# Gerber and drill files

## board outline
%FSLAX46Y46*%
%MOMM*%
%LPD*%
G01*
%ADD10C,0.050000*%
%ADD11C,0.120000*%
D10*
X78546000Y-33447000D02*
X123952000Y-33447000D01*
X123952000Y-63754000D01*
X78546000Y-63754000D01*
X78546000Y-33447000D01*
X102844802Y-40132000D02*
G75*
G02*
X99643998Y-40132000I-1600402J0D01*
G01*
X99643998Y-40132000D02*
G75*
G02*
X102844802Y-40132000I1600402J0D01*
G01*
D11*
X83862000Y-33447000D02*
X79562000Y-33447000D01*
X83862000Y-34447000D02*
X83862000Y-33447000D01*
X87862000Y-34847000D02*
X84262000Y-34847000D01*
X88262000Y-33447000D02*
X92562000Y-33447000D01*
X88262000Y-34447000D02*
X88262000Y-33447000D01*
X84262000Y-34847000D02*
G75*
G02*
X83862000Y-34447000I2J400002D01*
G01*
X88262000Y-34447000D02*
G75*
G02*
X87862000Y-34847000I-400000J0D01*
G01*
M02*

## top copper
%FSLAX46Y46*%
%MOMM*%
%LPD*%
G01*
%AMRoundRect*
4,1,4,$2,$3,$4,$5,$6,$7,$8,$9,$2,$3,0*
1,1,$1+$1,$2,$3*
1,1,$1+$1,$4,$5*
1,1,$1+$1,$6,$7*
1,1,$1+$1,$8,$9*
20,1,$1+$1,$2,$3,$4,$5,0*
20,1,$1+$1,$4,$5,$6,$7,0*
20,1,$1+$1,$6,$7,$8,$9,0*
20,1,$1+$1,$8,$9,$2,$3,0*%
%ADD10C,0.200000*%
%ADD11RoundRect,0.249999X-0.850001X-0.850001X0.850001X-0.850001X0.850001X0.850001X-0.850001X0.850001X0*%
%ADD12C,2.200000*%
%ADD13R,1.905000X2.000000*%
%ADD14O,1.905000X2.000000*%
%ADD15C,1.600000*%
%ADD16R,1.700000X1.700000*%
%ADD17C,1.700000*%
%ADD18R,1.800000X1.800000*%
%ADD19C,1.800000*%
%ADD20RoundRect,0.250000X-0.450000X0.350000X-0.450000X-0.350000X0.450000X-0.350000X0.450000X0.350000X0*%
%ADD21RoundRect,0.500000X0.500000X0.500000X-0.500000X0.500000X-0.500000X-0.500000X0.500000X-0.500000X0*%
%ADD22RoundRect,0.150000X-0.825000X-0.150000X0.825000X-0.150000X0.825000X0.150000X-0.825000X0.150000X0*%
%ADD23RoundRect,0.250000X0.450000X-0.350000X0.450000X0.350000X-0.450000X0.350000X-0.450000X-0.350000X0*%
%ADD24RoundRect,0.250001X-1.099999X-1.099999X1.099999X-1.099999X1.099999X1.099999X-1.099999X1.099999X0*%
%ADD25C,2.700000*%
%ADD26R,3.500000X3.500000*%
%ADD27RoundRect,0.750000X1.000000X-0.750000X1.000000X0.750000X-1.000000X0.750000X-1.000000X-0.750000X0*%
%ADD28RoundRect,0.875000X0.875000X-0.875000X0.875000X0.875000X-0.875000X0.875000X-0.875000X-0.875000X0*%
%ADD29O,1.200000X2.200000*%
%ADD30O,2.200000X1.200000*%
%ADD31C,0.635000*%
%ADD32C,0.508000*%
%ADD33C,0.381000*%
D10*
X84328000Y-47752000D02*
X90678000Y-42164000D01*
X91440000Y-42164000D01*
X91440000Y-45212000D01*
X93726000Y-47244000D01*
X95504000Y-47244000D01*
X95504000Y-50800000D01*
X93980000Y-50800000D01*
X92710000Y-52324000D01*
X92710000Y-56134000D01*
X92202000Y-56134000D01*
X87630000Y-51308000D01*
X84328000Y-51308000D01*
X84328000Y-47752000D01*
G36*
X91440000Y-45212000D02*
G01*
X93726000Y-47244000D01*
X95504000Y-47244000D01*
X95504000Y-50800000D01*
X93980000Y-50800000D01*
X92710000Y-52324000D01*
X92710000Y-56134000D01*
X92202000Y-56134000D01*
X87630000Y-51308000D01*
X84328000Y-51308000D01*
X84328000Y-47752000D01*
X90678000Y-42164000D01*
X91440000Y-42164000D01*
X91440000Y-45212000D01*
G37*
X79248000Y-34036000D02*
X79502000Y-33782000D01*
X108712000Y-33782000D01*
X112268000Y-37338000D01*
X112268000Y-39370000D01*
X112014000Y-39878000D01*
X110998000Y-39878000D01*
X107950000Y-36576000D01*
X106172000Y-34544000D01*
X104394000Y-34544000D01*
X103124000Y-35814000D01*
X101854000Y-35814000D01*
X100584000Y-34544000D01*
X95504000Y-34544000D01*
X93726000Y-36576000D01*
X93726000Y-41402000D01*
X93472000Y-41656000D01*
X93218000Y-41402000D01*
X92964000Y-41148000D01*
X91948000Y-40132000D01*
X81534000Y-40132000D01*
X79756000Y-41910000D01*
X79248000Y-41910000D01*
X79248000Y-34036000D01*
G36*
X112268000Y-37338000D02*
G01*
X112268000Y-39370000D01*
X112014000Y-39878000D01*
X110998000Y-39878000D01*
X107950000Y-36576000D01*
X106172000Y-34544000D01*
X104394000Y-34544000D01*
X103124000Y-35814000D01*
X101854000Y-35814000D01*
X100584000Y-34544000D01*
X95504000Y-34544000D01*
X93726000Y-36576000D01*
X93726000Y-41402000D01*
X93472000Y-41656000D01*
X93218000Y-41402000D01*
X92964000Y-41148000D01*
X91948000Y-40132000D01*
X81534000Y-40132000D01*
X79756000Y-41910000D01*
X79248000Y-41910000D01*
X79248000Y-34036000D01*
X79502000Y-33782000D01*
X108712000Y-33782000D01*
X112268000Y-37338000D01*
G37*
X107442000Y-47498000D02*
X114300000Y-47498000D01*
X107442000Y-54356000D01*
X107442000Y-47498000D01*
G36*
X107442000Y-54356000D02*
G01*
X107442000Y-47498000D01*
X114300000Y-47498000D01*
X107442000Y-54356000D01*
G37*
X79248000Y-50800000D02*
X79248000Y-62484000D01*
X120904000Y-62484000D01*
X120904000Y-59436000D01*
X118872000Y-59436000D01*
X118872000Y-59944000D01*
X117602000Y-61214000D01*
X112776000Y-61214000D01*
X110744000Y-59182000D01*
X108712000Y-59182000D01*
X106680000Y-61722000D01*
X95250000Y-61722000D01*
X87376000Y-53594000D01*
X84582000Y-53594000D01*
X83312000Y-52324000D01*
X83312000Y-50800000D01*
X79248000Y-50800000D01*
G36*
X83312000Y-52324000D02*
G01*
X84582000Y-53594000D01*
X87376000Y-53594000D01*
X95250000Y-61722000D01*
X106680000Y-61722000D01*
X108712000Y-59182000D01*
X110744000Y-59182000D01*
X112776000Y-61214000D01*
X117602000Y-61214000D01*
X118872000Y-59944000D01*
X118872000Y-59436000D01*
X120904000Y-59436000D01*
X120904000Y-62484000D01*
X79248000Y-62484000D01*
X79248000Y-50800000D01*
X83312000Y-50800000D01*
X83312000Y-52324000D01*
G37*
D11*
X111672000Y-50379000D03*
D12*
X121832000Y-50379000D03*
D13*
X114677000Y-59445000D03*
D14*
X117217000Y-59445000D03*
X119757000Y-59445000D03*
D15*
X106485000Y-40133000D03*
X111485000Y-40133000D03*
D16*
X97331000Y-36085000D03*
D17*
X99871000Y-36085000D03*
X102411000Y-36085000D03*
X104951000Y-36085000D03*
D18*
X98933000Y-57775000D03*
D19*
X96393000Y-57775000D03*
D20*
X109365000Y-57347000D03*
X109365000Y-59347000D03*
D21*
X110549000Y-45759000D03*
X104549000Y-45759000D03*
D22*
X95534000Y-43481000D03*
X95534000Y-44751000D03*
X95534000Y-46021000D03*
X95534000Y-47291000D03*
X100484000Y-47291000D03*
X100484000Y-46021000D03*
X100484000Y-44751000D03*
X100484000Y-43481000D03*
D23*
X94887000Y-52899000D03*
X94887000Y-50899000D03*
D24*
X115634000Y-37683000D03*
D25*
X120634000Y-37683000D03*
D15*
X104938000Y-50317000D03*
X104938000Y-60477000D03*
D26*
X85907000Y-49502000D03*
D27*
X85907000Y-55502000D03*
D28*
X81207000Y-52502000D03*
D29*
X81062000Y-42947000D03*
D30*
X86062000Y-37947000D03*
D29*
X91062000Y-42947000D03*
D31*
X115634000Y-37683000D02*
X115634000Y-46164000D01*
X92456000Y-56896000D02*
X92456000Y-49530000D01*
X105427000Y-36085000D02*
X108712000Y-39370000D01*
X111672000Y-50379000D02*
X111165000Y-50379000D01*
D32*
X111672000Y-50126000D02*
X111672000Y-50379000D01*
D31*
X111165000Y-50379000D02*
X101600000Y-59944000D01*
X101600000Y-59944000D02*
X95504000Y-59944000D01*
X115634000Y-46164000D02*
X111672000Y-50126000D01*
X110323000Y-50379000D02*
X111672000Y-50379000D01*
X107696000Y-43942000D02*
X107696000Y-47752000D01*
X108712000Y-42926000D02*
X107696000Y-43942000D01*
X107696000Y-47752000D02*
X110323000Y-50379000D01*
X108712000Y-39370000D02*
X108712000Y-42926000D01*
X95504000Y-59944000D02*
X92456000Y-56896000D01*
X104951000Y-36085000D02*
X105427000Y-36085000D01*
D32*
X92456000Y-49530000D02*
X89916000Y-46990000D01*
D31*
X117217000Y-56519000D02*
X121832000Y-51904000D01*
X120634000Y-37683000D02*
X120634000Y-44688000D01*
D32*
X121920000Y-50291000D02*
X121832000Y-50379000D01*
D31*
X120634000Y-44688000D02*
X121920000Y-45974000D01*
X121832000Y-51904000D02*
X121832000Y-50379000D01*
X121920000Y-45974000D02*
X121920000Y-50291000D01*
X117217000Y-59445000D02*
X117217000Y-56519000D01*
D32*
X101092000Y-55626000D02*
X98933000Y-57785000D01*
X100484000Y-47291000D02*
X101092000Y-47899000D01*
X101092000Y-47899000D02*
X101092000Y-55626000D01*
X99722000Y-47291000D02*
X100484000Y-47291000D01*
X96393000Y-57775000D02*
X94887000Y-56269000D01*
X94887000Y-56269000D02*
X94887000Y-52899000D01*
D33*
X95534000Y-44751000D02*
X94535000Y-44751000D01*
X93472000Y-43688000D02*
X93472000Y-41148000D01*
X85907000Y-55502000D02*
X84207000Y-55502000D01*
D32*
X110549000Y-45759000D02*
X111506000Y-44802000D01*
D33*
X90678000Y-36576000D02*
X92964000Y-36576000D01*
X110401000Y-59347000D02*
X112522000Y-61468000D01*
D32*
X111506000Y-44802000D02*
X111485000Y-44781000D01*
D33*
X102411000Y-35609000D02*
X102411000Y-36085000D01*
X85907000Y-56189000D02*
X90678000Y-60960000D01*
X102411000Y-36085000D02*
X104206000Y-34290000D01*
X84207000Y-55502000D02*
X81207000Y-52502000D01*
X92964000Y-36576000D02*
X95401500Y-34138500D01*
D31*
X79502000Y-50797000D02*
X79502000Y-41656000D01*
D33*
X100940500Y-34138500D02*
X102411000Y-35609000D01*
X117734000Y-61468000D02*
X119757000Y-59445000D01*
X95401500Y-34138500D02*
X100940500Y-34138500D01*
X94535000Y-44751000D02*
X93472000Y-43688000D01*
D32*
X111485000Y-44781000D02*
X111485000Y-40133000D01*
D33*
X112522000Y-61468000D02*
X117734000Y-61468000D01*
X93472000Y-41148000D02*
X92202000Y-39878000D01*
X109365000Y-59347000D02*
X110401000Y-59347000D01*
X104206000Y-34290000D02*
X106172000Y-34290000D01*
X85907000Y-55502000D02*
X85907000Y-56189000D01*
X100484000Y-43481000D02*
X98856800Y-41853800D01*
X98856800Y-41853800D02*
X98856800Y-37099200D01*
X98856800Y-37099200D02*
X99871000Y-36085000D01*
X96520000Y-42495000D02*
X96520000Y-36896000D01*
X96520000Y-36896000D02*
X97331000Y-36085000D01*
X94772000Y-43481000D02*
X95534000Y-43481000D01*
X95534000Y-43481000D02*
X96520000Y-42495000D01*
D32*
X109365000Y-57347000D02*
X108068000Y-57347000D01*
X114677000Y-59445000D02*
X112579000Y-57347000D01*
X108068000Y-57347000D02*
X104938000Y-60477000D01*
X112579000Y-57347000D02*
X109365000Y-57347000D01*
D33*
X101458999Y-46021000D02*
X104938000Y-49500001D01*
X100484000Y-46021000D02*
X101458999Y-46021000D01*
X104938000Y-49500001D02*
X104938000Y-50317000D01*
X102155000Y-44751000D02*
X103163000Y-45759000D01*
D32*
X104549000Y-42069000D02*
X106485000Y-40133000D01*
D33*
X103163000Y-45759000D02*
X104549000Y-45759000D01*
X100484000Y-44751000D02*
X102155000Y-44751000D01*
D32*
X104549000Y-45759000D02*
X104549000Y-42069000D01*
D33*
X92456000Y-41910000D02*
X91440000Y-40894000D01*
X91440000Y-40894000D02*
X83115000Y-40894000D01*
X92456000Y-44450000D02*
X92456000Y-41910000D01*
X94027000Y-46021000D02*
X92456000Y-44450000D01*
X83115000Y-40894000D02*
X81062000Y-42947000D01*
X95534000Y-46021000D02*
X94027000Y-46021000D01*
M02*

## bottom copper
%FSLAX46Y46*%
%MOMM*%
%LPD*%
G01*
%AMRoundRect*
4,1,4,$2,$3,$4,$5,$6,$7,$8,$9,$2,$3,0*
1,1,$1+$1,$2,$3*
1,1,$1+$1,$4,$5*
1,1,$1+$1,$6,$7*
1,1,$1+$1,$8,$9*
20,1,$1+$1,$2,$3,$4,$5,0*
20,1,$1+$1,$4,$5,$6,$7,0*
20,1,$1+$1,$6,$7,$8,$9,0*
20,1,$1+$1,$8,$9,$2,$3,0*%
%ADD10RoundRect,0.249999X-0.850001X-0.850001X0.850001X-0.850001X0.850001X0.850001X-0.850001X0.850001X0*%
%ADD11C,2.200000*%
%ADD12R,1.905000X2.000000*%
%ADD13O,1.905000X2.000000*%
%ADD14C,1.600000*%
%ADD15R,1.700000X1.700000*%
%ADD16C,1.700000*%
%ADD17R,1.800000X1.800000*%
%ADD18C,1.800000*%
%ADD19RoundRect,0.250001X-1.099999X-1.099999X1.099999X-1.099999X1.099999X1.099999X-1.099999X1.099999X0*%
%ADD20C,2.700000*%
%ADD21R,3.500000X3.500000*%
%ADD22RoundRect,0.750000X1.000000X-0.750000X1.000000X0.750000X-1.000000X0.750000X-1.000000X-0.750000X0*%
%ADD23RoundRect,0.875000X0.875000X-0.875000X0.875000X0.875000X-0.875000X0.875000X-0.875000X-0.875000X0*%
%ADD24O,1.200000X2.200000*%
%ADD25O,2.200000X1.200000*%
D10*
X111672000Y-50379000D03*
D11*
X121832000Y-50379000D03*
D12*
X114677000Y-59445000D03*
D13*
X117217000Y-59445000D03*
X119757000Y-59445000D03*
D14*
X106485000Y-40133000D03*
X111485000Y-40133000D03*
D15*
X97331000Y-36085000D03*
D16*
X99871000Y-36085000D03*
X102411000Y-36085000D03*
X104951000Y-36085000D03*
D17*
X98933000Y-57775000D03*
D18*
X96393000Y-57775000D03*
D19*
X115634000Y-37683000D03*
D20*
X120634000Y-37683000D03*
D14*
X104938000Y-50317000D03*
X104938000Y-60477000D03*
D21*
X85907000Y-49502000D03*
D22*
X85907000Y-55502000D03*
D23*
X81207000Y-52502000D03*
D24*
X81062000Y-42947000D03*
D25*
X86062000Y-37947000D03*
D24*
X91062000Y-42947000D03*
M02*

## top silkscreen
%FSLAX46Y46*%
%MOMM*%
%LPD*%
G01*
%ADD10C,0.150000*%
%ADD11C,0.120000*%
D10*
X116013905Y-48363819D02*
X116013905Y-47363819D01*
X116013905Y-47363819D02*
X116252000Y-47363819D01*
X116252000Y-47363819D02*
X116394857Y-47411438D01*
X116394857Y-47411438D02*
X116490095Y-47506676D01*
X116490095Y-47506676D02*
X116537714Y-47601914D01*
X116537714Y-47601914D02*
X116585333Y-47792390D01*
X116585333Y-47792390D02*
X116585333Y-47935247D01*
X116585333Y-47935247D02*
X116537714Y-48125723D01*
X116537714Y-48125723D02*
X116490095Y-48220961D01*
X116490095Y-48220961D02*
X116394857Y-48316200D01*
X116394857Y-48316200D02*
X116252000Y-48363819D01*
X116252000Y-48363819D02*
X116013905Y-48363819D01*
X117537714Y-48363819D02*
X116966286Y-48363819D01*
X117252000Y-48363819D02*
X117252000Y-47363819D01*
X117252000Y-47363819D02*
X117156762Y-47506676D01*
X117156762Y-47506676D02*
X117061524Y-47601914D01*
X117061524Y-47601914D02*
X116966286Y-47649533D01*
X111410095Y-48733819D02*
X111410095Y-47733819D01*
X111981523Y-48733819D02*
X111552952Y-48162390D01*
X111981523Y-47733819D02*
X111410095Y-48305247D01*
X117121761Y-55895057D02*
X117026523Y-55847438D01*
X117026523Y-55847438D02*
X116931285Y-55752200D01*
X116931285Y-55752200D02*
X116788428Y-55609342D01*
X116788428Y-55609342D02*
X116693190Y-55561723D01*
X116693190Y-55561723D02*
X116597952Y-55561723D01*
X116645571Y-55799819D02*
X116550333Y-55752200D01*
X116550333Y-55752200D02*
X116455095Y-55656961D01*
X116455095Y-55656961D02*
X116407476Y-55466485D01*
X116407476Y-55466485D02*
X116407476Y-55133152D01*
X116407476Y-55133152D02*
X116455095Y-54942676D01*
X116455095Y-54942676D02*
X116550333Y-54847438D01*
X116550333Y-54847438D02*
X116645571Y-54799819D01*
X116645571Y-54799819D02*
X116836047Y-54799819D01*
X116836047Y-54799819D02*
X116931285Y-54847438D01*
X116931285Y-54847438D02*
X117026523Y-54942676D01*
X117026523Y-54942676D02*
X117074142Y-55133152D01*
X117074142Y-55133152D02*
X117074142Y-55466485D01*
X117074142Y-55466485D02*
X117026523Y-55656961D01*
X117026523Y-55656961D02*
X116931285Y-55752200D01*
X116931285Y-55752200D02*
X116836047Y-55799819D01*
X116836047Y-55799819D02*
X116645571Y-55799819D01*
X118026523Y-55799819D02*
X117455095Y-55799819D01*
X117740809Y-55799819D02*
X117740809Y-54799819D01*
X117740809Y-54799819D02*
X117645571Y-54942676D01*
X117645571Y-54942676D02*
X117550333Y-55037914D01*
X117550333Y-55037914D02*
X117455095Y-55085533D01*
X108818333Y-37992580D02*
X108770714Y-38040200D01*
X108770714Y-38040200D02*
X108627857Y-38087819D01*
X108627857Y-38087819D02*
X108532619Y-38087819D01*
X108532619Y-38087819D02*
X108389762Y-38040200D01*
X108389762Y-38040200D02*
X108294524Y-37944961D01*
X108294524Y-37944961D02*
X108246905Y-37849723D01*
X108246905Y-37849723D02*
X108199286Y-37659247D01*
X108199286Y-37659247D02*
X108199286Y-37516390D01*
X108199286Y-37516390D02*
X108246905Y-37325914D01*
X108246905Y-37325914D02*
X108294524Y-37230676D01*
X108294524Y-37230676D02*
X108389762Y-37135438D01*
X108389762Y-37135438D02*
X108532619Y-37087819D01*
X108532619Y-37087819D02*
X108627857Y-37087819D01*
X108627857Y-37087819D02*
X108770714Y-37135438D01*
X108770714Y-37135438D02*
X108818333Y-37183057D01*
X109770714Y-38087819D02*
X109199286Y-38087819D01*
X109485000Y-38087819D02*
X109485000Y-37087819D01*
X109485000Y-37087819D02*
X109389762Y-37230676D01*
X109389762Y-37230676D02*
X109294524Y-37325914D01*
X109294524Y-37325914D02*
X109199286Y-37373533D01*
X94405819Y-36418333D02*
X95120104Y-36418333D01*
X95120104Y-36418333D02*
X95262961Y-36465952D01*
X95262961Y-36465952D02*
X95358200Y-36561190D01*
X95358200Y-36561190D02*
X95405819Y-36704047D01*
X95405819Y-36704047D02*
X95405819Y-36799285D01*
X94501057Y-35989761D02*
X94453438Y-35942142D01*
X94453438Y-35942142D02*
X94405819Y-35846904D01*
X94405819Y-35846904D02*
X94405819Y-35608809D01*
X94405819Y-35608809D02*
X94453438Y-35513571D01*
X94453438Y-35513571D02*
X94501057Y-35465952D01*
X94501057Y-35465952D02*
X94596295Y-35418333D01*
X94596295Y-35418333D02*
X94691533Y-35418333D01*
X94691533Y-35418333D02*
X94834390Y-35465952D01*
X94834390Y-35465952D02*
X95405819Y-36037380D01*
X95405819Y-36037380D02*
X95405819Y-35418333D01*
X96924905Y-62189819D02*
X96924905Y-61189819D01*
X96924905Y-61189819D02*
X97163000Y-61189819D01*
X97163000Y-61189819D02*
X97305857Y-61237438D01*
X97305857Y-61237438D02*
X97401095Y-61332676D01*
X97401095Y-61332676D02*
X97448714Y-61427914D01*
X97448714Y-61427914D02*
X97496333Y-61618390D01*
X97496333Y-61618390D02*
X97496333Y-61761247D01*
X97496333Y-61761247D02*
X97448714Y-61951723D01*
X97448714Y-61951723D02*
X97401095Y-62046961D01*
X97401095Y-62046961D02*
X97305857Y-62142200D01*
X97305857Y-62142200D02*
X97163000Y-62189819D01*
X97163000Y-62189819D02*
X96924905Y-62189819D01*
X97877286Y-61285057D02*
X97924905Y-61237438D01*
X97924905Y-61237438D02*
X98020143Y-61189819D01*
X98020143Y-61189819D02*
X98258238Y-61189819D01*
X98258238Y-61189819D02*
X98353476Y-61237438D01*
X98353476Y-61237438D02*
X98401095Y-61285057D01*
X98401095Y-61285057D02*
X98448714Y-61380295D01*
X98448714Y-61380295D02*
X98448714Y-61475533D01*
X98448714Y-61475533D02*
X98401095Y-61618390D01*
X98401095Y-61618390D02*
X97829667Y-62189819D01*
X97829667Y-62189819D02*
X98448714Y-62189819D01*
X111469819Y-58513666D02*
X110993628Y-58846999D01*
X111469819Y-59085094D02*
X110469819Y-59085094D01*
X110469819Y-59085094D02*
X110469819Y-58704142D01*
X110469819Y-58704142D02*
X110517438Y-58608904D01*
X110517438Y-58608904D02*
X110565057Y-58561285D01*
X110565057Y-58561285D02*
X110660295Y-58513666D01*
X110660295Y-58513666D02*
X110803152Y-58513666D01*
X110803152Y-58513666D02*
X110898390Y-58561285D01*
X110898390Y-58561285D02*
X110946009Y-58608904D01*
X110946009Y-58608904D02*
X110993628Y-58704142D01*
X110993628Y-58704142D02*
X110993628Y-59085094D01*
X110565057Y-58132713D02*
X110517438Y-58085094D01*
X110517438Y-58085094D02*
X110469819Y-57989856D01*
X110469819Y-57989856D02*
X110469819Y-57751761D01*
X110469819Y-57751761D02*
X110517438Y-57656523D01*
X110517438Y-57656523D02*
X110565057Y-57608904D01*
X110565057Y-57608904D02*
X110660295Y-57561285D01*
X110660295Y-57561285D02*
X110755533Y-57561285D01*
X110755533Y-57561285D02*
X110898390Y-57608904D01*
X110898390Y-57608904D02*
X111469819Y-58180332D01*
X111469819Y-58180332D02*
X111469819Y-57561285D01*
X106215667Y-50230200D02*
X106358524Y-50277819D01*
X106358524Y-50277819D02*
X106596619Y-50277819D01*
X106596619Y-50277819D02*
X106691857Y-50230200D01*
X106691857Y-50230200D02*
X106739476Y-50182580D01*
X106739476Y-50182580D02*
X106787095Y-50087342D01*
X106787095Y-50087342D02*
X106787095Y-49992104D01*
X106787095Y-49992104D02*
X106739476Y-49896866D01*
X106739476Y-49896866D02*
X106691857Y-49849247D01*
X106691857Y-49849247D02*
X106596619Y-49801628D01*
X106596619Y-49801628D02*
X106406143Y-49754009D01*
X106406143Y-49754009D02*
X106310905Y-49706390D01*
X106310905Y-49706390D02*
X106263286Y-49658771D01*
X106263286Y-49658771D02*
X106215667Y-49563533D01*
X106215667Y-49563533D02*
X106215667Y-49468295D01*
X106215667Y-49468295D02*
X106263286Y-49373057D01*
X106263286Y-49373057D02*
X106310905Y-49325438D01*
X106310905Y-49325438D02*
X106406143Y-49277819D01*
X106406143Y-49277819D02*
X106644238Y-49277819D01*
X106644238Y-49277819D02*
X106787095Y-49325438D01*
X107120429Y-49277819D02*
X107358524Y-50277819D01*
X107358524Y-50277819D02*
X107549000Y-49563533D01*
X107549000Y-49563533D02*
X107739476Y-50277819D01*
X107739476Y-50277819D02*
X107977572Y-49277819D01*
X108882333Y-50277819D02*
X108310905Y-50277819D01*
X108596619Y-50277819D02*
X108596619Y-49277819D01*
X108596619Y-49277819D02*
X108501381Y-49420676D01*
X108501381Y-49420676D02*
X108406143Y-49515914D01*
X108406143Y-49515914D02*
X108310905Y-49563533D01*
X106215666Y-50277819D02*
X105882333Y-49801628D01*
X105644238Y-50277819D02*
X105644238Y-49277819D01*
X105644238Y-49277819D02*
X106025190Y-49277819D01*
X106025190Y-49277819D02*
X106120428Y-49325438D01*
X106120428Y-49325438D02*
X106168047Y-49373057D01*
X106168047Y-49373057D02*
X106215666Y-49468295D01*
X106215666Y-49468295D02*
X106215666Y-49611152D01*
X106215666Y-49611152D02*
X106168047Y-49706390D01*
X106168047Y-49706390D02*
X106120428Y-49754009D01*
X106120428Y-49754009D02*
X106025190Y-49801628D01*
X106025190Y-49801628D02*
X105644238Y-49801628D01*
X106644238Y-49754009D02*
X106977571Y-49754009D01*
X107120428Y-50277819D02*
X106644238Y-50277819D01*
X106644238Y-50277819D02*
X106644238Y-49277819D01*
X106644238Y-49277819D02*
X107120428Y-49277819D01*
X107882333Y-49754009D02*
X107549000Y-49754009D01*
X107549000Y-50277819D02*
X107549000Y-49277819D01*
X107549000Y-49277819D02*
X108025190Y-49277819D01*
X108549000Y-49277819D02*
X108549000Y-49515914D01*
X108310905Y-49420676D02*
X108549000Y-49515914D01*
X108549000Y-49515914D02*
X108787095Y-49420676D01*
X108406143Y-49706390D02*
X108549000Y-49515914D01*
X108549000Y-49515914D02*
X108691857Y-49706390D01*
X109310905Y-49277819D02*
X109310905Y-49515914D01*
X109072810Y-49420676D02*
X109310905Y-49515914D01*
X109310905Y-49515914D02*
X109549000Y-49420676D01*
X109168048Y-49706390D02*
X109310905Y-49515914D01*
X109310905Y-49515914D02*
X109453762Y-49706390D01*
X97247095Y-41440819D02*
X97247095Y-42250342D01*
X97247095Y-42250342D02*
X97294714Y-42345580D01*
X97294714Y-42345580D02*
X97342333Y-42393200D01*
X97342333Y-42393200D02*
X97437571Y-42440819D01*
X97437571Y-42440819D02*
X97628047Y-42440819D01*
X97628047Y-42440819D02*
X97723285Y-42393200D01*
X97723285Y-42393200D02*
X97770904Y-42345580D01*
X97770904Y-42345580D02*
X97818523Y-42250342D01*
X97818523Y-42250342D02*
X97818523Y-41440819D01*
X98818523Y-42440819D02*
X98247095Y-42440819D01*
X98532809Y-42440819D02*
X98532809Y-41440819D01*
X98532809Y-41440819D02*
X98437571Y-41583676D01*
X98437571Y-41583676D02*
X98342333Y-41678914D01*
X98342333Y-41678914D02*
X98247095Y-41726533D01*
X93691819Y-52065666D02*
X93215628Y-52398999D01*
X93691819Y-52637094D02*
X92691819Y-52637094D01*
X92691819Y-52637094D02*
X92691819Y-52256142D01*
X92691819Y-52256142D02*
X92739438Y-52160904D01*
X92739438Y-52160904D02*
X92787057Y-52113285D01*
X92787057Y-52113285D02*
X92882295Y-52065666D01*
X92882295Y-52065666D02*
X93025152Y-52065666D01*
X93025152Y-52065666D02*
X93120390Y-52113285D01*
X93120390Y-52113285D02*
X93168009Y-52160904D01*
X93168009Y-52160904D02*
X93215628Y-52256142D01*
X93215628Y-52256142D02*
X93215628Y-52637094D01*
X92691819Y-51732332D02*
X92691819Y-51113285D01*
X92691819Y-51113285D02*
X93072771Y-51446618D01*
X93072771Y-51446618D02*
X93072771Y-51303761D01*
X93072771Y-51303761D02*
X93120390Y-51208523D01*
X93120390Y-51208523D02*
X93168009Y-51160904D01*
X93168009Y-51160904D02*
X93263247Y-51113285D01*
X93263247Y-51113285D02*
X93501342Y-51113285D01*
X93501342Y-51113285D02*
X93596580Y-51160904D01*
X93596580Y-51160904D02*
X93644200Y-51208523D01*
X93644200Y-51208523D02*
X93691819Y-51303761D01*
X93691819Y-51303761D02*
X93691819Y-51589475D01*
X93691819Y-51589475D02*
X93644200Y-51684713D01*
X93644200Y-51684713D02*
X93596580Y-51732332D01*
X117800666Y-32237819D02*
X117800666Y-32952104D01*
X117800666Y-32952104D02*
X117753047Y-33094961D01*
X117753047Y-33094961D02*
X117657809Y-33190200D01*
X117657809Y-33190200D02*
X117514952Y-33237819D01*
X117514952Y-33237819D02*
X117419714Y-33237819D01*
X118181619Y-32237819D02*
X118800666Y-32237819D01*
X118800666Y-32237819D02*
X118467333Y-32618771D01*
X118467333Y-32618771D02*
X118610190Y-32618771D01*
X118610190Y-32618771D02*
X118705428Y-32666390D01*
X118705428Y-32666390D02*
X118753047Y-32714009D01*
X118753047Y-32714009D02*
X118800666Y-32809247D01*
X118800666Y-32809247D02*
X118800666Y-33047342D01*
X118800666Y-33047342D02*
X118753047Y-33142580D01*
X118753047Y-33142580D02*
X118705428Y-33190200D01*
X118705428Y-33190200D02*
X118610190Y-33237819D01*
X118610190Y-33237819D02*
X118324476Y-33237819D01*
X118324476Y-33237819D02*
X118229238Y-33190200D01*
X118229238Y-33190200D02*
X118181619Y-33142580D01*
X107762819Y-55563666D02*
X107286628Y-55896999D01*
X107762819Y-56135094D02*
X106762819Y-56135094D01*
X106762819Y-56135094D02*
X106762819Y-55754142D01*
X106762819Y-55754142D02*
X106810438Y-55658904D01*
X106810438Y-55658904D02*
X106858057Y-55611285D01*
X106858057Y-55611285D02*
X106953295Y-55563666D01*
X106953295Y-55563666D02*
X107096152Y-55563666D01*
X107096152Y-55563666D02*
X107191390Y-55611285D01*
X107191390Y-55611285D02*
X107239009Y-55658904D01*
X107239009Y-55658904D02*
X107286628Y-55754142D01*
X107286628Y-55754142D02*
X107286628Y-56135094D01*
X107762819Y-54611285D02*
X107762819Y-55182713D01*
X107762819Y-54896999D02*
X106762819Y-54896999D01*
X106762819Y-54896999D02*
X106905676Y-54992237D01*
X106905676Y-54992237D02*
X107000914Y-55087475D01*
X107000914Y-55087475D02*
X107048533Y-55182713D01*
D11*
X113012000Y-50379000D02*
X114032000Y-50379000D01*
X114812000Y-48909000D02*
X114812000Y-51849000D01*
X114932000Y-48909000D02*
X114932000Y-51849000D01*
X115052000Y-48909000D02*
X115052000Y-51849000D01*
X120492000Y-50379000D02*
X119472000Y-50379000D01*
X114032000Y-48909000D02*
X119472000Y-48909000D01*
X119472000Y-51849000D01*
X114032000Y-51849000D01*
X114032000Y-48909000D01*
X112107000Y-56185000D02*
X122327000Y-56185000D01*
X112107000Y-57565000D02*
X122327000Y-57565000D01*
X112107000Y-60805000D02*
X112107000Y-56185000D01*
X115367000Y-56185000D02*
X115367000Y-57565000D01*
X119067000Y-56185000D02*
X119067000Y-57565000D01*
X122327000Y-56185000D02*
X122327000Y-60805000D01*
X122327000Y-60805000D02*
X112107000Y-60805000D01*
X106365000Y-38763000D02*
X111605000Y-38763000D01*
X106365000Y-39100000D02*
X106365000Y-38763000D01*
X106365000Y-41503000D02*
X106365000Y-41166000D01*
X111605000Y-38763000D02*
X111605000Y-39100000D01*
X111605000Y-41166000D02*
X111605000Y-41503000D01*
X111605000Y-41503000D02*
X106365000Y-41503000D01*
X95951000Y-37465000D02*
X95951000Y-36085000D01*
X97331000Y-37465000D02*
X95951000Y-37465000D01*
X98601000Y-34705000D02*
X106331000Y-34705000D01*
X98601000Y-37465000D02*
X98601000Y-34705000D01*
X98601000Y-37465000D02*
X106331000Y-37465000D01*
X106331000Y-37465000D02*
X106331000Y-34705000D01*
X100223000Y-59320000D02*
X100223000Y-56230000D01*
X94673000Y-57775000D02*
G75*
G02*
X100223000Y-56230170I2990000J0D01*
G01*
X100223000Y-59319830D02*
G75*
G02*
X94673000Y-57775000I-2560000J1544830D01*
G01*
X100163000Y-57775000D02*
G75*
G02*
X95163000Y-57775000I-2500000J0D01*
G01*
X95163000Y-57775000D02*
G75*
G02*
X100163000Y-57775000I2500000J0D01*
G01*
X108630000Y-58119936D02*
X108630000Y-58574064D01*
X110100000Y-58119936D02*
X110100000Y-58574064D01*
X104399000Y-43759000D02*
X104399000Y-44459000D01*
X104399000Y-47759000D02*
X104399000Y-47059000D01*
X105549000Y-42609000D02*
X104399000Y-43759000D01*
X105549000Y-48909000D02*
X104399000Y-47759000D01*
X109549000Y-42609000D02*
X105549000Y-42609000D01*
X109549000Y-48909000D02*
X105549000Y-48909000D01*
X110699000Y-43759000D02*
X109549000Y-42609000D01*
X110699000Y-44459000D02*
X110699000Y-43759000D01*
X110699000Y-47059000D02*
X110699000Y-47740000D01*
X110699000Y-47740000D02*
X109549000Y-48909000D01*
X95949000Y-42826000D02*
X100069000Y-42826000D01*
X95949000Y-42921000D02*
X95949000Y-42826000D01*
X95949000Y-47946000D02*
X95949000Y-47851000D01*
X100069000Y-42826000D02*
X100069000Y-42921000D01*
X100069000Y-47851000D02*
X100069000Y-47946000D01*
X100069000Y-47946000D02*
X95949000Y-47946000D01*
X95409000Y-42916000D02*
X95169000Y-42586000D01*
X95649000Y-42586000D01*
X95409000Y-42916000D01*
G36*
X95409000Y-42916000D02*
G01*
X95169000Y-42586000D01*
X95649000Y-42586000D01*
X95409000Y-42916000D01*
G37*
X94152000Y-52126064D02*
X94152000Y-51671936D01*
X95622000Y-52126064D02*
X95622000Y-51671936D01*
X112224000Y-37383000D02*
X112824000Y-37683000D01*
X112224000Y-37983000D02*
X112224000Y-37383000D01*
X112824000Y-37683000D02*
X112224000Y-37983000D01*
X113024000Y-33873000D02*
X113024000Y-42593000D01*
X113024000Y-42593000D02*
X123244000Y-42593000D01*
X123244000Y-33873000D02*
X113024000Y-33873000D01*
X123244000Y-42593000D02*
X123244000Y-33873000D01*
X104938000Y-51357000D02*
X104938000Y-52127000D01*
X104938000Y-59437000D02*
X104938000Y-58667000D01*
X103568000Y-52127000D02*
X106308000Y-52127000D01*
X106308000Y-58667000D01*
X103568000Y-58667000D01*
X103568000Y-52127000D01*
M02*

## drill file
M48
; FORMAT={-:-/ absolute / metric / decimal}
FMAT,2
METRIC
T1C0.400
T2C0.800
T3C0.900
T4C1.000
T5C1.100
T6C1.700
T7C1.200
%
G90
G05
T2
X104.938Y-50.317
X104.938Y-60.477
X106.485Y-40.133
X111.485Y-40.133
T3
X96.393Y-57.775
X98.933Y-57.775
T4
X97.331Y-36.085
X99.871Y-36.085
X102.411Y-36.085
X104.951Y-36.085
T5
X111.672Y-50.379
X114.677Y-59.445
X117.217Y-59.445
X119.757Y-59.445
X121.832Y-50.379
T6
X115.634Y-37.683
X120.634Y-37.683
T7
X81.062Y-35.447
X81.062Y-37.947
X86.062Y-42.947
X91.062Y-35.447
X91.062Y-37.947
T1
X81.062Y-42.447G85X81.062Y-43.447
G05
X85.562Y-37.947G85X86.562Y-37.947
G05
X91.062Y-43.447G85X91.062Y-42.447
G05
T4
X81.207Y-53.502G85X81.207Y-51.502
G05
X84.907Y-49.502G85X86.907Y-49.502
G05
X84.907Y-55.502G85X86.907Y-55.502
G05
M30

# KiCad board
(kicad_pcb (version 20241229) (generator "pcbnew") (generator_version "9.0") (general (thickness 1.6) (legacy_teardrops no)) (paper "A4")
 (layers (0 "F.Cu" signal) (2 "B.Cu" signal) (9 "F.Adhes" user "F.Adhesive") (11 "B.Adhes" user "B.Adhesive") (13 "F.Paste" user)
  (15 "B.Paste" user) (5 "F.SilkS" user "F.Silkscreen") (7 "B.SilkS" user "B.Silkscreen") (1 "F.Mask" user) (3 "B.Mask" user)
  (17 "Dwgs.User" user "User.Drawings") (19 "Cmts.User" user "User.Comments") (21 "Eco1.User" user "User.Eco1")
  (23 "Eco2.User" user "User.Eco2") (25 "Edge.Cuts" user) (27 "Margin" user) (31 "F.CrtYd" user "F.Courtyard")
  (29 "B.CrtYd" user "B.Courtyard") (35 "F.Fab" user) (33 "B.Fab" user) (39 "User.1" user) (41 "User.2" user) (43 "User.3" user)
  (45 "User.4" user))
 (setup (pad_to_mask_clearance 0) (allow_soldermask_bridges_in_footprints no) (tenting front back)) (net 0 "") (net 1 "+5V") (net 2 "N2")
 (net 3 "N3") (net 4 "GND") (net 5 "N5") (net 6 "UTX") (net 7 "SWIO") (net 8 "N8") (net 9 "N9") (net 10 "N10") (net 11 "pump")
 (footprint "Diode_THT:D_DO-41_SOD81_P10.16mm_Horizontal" (layer "F.Cu") (at 111.672 50.379)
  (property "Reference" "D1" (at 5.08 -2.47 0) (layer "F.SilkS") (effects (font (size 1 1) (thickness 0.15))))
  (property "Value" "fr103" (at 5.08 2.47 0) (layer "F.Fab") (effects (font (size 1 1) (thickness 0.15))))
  (fp_line (start 1.34 0) (end 2.36 0) (stroke (width 0.12) (type solid)) (layer "F.SilkS"))
  (fp_line (start 3.14 -1.47) (end 3.14 1.47) (stroke (width 0.12) (type solid)) (layer "F.SilkS"))
  (fp_line (start 3.26 -1.47) (end 3.26 1.47) (stroke (width 0.12) (type solid)) (layer "F.SilkS"))
  (fp_line (start 3.38 -1.47) (end 3.38 1.47) (stroke (width 0.12) (type solid)) (layer "F.SilkS"))
  (fp_line (start 8.82 0) (end 7.8 0) (stroke (width 0.12) (type solid)) (layer "F.SilkS"))
  (fp_rect (start 2.36 -1.47) (end 7.8 1.47) (stroke (width 0.12) (type solid)) (fill no) (layer "F.SilkS"))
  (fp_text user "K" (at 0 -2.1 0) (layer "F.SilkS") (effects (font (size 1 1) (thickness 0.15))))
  (pad "1" thru_hole roundrect (at 0 0) (size 2.2 2.2) (drill 1.1) (layers "*.Cu" "*.Mask") (remove_unused_layers no)
   (roundrect_rratio 0.113636) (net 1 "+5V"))
  (pad "2" thru_hole circle (at 10.16 0) (size 2.2 2.2) (drill 1.1) (layers "*.Cu" "*.Mask") (remove_unused_layers no) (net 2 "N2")))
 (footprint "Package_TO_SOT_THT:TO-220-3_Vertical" (layer "F.Cu") (at 114.677 59.445)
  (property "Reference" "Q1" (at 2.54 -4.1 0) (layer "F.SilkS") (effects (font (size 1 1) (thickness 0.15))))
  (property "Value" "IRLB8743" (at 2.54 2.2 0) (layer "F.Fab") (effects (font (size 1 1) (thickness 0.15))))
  (fp_line (start -2.57 -3.26) (end 7.65 -3.26) (stroke (width 0.12) (type solid)) (layer "F.SilkS"))
  (fp_line (start -2.57 -1.88) (end 7.65 -1.88) (stroke (width 0.12) (type solid)) (layer "F.SilkS"))
  (fp_line (start -2.57 1.36) (end -2.57 -3.26) (stroke (width 0.12) (type solid)) (layer "F.SilkS"))
  (fp_line (start 0.69 -3.26) (end 0.69 -1.88) (stroke (width 0.12) (type solid)) (layer "F.SilkS"))
  (fp_line (start 4.39 -3.26) (end 4.39 -1.88) (stroke (width 0.12) (type solid)) (layer "F.SilkS"))
  (fp_line (start 7.65 -3.26) (end 7.65 1.36) (stroke (width 0.12) (type solid)) (layer "F.SilkS"))
  (fp_line (start 7.65 1.36) (end -2.57 1.36) (stroke (width 0.12) (type solid)) (layer "F.SilkS"))
  (pad "1" thru_hole rect (at 0 0) (size 1.905 2) (drill 1.1) (layers "*.Cu" "*.Mask") (remove_unused_layers no) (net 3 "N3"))
  (pad "2" thru_hole oval (at 2.54 0) (size 1.905 2) (drill 1.1) (layers "*.Cu" "*.Mask") (remove_unused_layers no) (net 2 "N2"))
  (pad "3" thru_hole oval (at 5.08 0) (size 1.905 2) (drill 1.1) (layers "*.Cu" "*.Mask") (remove_unused_layers no) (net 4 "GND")))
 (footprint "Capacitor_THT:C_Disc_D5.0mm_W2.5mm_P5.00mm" (layer "F.Cu") (at 106.485 40.133)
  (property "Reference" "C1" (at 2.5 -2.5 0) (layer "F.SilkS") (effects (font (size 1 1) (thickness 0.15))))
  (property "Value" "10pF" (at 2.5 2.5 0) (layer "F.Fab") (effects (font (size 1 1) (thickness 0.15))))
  (fp_line (start -0.12 -1.37) (end 5.12 -1.37) (stroke (width 0.12) (type solid)) (layer "F.SilkS"))
  (fp_line (start -0.12 -1.033) (end -0.12 -1.37) (stroke (width 0.12) (type solid)) (layer "F.SilkS"))
  (fp_line (start -0.12 1.37) (end -0.12 1.033) (stroke (width 0.12) (type solid)) (layer "F.SilkS"))
  (fp_line (start 5.12 -1.37) (end 5.12 -1.033) (stroke (width 0.12) (type solid)) (layer "F.SilkS"))
  (fp_line (start 5.12 1.033) (end 5.12 1.37) (stroke (width 0.12) (type solid)) (layer "F.SilkS"))
  (fp_line (start 5.12 1.37) (end -0.12 1.37) (stroke (width 0.12) (type solid)) (layer "F.SilkS"))
  (pad "1" thru_hole circle (at 0 0) (size 1.6 1.6) (drill 0.8) (layers "*.Cu" "*.Mask") (remove_unused_layers no) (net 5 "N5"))
  (pad "2" thru_hole circle (at 5 0) (size 1.6 1.6) (drill 0.8) (layers "*.Cu" "*.Mask") (remove_unused_layers no) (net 4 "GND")))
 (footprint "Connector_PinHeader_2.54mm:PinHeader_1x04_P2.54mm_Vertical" (layer "F.Cu") (at 97.331 36.085 90)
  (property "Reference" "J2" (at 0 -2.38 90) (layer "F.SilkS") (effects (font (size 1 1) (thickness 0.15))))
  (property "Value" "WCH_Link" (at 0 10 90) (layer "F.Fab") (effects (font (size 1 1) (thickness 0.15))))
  (fp_line (start -1.38 -1.38) (end 0 -1.38) (stroke (width 0.12) (type solid)) (layer "F.SilkS"))
  (fp_line (start -1.38 0) (end -1.38 -1.38) (stroke (width 0.12) (type solid)) (layer "F.SilkS"))
  (fp_line (start 1.38 1.27) (end 1.38 9) (stroke (width 0.12) (type solid)) (layer "F.SilkS"))
  (fp_line (start -1.38 1.27) (end 1.38 1.27) (stroke (width 0.12) (type solid)) (layer "F.SilkS"))
  (fp_line (start -1.38 1.27) (end -1.38 9) (stroke (width 0.12) (type solid)) (layer "F.SilkS"))
  (fp_line (start -1.38 9) (end 1.38 9) (stroke (width 0.12) (type solid)) (layer "F.SilkS"))
  (pad "1" thru_hole rect (at 0 0 90) (size 1.7 1.7) (drill 1) (layers "*.Cu" "*.Mask") (remove_unused_layers no) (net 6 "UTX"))
  (pad "2" thru_hole circle (at 0 2.54 90) (size 1.7 1.7) (drill 1) (layers "*.Cu" "*.Mask") (remove_unused_layers no) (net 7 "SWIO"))
  (pad "3" thru_hole circle (at 0 5.08 90) (size 1.7 1.7) (drill 1) (layers "*.Cu" "*.Mask") (remove_unused_layers no) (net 4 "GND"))
  (pad "4" thru_hole circle (at 0 7.62 90) (size 1.7 1.7) (drill 1) (layers "*.Cu" "*.Mask") (remove_unused_layers no) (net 1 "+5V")))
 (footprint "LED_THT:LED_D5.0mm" (layer "F.Cu") (at 98.933 57.775 180)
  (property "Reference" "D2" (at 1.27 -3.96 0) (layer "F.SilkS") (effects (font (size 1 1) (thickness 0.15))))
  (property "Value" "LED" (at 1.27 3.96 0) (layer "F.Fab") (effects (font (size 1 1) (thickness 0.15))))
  (fp_line (start -1.29 -1.545) (end -1.29 1.545) (stroke (width 0.12) (type solid)) (layer "F.SilkS"))
  (fp_arc (start 4.26 0) (mid 2.071779 2.880495) (end -1.29 1.54483) (stroke (width 0.12) (type solid)) (layer "F.SilkS"))
  (fp_arc (start -1.29 -1.54483) (mid 2.071779 -2.880495) (end 4.26 0) (stroke (width 0.12) (type solid)) (layer "F.SilkS"))
  (fp_circle (center 1.27 0) (end 3.77 0) (stroke (width 0.12) (type solid)) (fill no) (layer "F.SilkS"))
  (pad "1" thru_hole rect (at 0 0 180) (size 1.8 1.8) (drill 0.9) (layers "*.Cu" "*.Mask") (remove_unused_layers no) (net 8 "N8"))
  (pad "2" thru_hole circle (at 2.54 0 180) (size 1.8 1.8) (drill 0.9) (layers "*.Cu" "*.Mask") (remove_unused_layers no) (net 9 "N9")))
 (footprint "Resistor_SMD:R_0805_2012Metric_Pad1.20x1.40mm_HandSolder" (layer "F.Cu") (at 109.365 58.347 -90)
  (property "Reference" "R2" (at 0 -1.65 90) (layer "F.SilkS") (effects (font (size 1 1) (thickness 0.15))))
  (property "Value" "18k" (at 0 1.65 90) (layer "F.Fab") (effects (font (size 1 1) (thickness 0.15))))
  (fp_line (start -0.227064 0.735) (end 0.227064 0.735) (stroke (width 0.12) (type solid)) (layer "F.SilkS"))
  (fp_line (start -0.227064 -0.735) (end 0.227064 -0.735) (stroke (width 0.12) (type solid)) (layer "F.SilkS"))
  (pad "1" smd roundrect (at -1 0 270) (size 1.2 1.4) (layers "F.Cu" "F.Mask" "F.Paste") (roundrect_rratio 0.208333) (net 3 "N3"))
  (pad "2" smd roundrect (at 1 0 270) (size 1.2 1.4) (layers "F.Cu" "F.Mask" "F.Paste") (roundrect_rratio 0.208333) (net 4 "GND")))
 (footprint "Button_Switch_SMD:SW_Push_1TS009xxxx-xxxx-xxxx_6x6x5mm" (layer "F.Cu") (at 107.549 45.759 180)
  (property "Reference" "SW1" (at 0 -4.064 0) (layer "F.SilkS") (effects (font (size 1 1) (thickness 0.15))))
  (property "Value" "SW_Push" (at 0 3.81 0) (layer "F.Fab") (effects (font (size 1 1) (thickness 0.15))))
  (fp_line (start 3.15 2) (end 3.15 1.3) (stroke (width 0.12) (type default)) (layer "F.SilkS"))
  (fp_line (start 3.15 -2) (end 3.15 -1.3) (stroke (width 0.12) (type default)) (layer "F.SilkS"))
  (fp_line (start 2 3.15) (end 3.15 2) (stroke (width 0.12) (type default)) (layer "F.SilkS"))
  (fp_line (start 2 -3.15) (end 3.15 -2) (stroke (width 0.12) (type default)) (layer "F.SilkS"))
  (fp_line (start -2 3.15) (end 2 3.15) (stroke (width 0.12) (type default)) (layer "F.SilkS"))
  (fp_line (start -2 -3.15) (end 2 -3.15) (stroke (width 0.12) (type default)) (layer "F.SilkS"))
  (fp_line (start -3.15 2) (end -2 3.15) (stroke (width 0.12) (type default)) (layer "F.SilkS"))
  (fp_line (start -3.15 1.3) (end -3.15 2) (stroke (width 0.12) (type default)) (layer "F.SilkS"))
  (fp_line (start -3.15 -1.3) (end -3.15 -1.981) (stroke (width 0.12) (type default)) (layer "F.SilkS"))
  (fp_line (start -3.15 -1.981) (end -2 -3.15) (stroke (width 0.12) (type default)) (layer "F.SilkS"))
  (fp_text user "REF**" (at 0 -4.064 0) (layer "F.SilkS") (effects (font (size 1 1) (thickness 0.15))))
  (pad "1" smd roundrect (at -3 0 180) (size 2 2) (layers "F.Cu" "F.Mask" "F.Paste") (roundrect_rratio 0.25) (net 4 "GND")
   (thermal_bridge_angle 45))
  (pad "2" smd roundrect (at 3 0 180) (size 2 2) (layers "F.Cu" "F.Mask" "F.Paste") (roundrect_rratio 0.25) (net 5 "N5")
   (thermal_bridge_angle 45)))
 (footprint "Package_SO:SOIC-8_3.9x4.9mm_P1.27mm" (layer "F.Cu") (at 98.009 45.386)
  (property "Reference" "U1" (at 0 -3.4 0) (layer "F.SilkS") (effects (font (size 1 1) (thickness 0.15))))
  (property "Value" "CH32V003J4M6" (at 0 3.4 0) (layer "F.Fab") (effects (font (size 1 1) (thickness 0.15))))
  (fp_line (start -2.06 -2.56) (end 2.06 -2.56) (stroke (width 0.12) (type solid)) (layer "F.SilkS"))
  (fp_line (start -2.06 -2.465) (end -2.06 -2.56) (stroke (width 0.12) (type solid)) (layer "F.SilkS"))
  (fp_line (start -2.06 2.56) (end -2.06 2.465) (stroke (width 0.12) (type solid)) (layer "F.SilkS"))
  (fp_line (start 2.06 -2.56) (end 2.06 -2.465) (stroke (width 0.12) (type solid)) (layer "F.SilkS"))
  (fp_line (start 2.06 2.465) (end 2.06 2.56) (stroke (width 0.12) (type solid)) (layer "F.SilkS"))
  (fp_line (start 2.06 2.56) (end -2.06 2.56) (stroke (width 0.12) (type solid)) (layer "F.SilkS"))
  (fp_poly (pts (xy -2.6 -2.47) (xy -2.84 -2.8) (xy -2.36 -2.8)) (stroke (width 0.12) (type solid)) (fill yes) (layer "F.SilkS"))
  (pad "1" smd roundrect (at -2.475 -1.905) (size 1.95 0.6) (layers "F.Cu" "F.Mask" "F.Paste") (roundrect_rratio 0.25) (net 6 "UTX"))
  (pad "2" smd roundrect (at -2.475 -0.635) (size 1.95 0.6) (layers "F.Cu" "F.Mask" "F.Paste") (roundrect_rratio 0.25) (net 4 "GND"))
  (pad "3" smd roundrect (at -2.475 0.635) (size 1.95 0.6) (layers "F.Cu" "F.Mask" "F.Paste") (roundrect_rratio 0.25) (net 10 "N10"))
  (pad "4" smd roundrect (at -2.475 1.905) (size 1.95 0.6) (layers "F.Cu" "F.Mask" "F.Paste") (roundrect_rratio 0.25) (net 1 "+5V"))
  (pad "5" smd roundrect (at 2.475 1.905) (size 1.95 0.6) (layers "F.Cu" "F.Mask" "F.Paste") (roundrect_rratio 0.25) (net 8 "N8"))
  (pad "6" smd roundrect (at 2.475 0.635) (size 1.95 0.6) (layers "F.Cu" "F.Mask" "F.Paste") (roundrect_rratio 0.25) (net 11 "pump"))
  (pad "7" smd roundrect (at 2.475 -0.635) (size 1.95 0.6) (layers "F.Cu" "F.Mask" "F.Paste") (roundrect_rratio 0.25) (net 5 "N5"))
  (pad "8" smd roundrect (at 2.475 -1.905) (size 1.95 0.6) (layers "F.Cu" "F.Mask" "F.Paste") (roundrect_rratio 0.25) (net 7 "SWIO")))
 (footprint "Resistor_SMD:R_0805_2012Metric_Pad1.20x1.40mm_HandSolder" (layer "F.Cu") (at 94.887 51.899 90)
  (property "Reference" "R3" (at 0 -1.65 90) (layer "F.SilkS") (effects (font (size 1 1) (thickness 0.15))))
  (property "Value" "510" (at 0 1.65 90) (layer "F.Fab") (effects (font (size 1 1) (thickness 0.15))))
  (fp_line (start -0.227064 -0.735) (end 0.227064 -0.735) (stroke (width 0.12) (type solid)) (layer "F.SilkS"))
  (fp_line (start -0.227064 0.735) (end 0.227064 0.735) (stroke (width 0.12) (type solid)) (layer "F.SilkS"))
  (pad "1" smd roundrect (at -1 0 90) (size 1.2 1.4) (layers "F.Cu" "F.Mask" "F.Paste") (roundrect_rratio 0.208333) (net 9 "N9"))
  (pad "2" smd roundrect (at 1 0 90) (size 1.2 1.4) (layers "F.Cu" "F.Mask" "F.Paste") (roundrect_rratio 0.208333) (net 1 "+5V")))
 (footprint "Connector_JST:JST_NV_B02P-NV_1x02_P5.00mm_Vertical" (layer "F.Cu") (at 115.634 37.683)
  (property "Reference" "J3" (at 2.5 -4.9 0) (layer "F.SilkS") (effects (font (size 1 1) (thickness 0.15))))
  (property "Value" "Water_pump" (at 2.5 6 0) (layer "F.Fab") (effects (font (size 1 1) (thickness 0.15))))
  (fp_line (start -3.41 -0.3) (end -2.81 0) (stroke (width 0.12) (type solid)) (layer "F.SilkS"))
  (fp_line (start -3.41 0.3) (end -3.41 -0.3) (stroke (width 0.12) (type solid)) (layer "F.SilkS"))
  (fp_line (start -2.81 0) (end -3.41 0.3) (stroke (width 0.12) (type solid)) (layer "F.SilkS"))
  (fp_line (start -2.61 -3.81) (end -2.61 4.91) (stroke (width 0.12) (type solid)) (layer "F.SilkS"))
  (fp_line (start -2.61 4.91) (end 7.61 4.91) (stroke (width 0.12) (type solid)) (layer "F.SilkS"))
  (fp_line (start 7.61 -3.81) (end -2.61 -3.81) (stroke (width 0.12) (type solid)) (layer "F.SilkS"))
  (fp_line (start 7.61 4.91) (end 7.61 -3.81) (stroke (width 0.12) (type solid)) (layer "F.SilkS"))
  (pad "1" thru_hole roundrect (at 0 0) (size 2.7 2.7) (drill 1.7) (layers "*.Cu" "*.Mask") (remove_unused_layers no)
   (roundrect_rratio 0.092593) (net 1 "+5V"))
  (pad "2" thru_hole circle (at 5 0) (size 2.7 2.7) (drill 1.7) (layers "*.Cu" "*.Mask") (remove_unused_layers no) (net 2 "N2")))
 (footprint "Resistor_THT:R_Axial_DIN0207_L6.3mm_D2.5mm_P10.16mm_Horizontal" (layer "F.Cu") (at 104.938 50.317 -90)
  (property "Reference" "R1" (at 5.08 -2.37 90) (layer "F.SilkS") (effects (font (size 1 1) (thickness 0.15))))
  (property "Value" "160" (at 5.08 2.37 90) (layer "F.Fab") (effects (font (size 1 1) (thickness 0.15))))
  (fp_line (start 1.04 0) (end 1.81 0) (stroke (width 0.12) (type solid)) (layer "F.SilkS"))
  (fp_line (start 9.12 0) (end 8.35 0) (stroke (width 0.12) (type solid)) (layer "F.SilkS"))
  (fp_rect (start 1.81 -1.37) (end 8.35 1.37) (stroke (width 0.12) (type solid)) (fill no) (layer "F.SilkS"))
  (pad "1" thru_hole circle (at 0 0 270) (size 1.6 1.6) (drill 0.8) (layers "*.Cu" "*.Mask") (remove_unused_layers no) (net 11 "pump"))
  (pad "2" thru_hole circle (at 10.16 0 270) (size 1.6 1.6) (drill 0.8) (layers "*.Cu" "*.Mask") (remove_unused_layers no) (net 3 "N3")))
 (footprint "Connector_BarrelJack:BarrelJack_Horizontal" (layer "B.Cu") (at 85.907 49.502 90)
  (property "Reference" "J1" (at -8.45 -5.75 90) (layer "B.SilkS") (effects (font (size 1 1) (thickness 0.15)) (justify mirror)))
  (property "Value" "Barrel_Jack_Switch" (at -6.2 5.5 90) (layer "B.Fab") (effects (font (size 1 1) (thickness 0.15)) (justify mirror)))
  (pad "1" thru_hole rect (at 0 0 90) (size 3.5 3.5) (drill oval 1 3) (layers "*.Cu" "*.Mask") (remove_unused_layers no) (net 1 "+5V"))
  (pad "2" thru_hole roundrect (at -6 0 90) (size 3 3.5) (drill oval 1 3) (layers "*.Cu" "*.Mask") (remove_unused_layers no)
   (roundrect_rratio 0.25) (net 4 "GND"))
  (pad "3" thru_hole roundrect (at -3 -4.7 90) (size 3.5 3.5) (drill oval 3 1) (layers "*.Cu" "*.Mask") (remove_unused_layers no)
   (roundrect_rratio 0.25) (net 4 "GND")))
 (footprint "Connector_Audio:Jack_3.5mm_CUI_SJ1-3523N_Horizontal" (layer "B.Cu") (at 86.062 37.947)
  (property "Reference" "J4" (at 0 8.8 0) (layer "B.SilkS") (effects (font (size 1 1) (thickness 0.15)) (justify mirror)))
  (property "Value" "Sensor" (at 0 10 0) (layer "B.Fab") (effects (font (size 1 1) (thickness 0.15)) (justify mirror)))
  (fp_line (start -2.2 -4.5) (end -6.5 -4.5) (stroke (width 0.12) (type solid)) (layer "Edge.Cuts"))
  (fp_line (start -2.2 -3.5) (end -2.2 -4.5) (stroke (width 0.12) (type solid)) (layer "Edge.Cuts"))
  (fp_line (start 1.8 -3.1) (end -1.8 -3.1) (stroke (width 0.12) (type solid)) (layer "Edge.Cuts"))
  (fp_line (start 2.2 -4.5) (end 6.5 -4.5) (stroke (width 0.12) (type solid)) (layer "Edge.Cuts"))
  (fp_line (start 2.2 -3.5) (end 2.2 -4.5) (stroke (width 0.12) (type solid)) (layer "Edge.Cuts"))
  (fp_arc (start -1.8 -3.1) (mid -2.082842 -3.217158) (end -2.2 -3.5) (stroke (width 0.12) (type solid)) (layer "Edge.Cuts"))
  (fp_arc (start 2.2 -3.5) (mid 2.082843 -3.217157) (end 1.8 -3.1) (stroke (width 0.12) (type solid)) (layer "Edge.Cuts"))
  (pad "" np_thru_hole circle (at -5 -2.5) (size 1.2 1.2) (drill 1.2) (layers "*.Cu" "*.Mask"))
  (pad "" np_thru_hole circle (at -5 0) (size 1.2 1.2) (drill 1.2) (layers "*.Cu" "*.Mask"))
  (pad "" np_thru_hole circle (at 0 5) (size 1.2 1.2) (drill 1.2) (layers "*.Cu" "*.Mask"))
  (pad "" np_thru_hole circle (at 5 -2.5) (size 1.2 1.2) (drill 1.2) (layers "*.Cu" "*.Mask"))
  (pad "" np_thru_hole circle (at 5 0) (size 1.2 1.2) (drill 1.2) (layers "*.Cu" "*.Mask"))
  (pad "R" thru_hole oval (at -5 5) (size 1.2 2.2) (drill oval 0.4 1.4) (layers "*.Cu" "*.Mask") (remove_unused_layers no) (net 10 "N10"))
  (pad "S" thru_hole oval (at 0 0) (size 2.2 1.2) (drill oval 1.4 0.4) (layers "*.Cu" "*.Mask") (remove_unused_layers no) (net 4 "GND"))
  (pad "T" thru_hole oval (at 5 5 180) (size 1.2 2.2) (drill oval 0.4 1.4) (layers "*.Cu" "*.Mask") (remove_unused_layers no) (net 1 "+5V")))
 (gr_poly
  (pts (xy 84.328 47.752) (xy 90.678 42.164) (xy 91.44 42.164) (xy 91.44 45.212) (xy 93.726 47.244) (xy 95.504 47.244) (xy 95.504 50.8)
   (xy 93.98 50.8) (xy 92.71 52.324) (xy 92.71 56.134) (xy 92.202 56.134) (xy 87.63 51.308) (xy 84.328 51.308))
  (stroke (width 0.2) (type solid)) (fill yes) (layer "F.Cu") (net 1))
 (gr_poly
  (pts (xy 79.248 34.036) (xy 79.502 33.782) (xy 108.712 33.782) (xy 112.268 37.338) (xy 112.268 39.37) (xy 112.014 39.878)
   (xy 110.998 39.878) (xy 107.95 36.576) (xy 106.172 34.544) (xy 104.394 34.544) (xy 103.124 35.814) (xy 101.854 35.814)
   (xy 100.584 34.544) (xy 95.504 34.544) (xy 93.726 36.576) (xy 93.726 41.402) (xy 93.472 41.656) (xy 93.218 41.402) (xy 92.964 41.148)
   (xy 91.948 40.132) (xy 81.534 40.132) (xy 79.756 41.91) (xy 79.248 41.91))
  (stroke (width 0.2) (type solid)) (fill yes) (layer "F.Cu") (net 4))
 (gr_poly
  (pts (xy 107.442 47.498) (xy 114.3 47.498) (xy 107.442 54.356)) (stroke (width 0.2) (type solid)) (fill yes) (layer "F.Cu") (net 1))
 (gr_poly
  (pts (xy 79.248 50.8) (xy 79.248 62.484) (xy 120.904 62.484) (xy 120.904 59.436) (xy 118.872 59.436) (xy 118.872 59.944)
   (xy 117.602 61.214) (xy 112.776 61.214) (xy 110.744 59.182) (xy 108.712 59.182) (xy 106.68 61.722) (xy 95.25 61.722) (xy 87.376 53.594)
   (xy 84.582 53.594) (xy 83.312 52.324) (xy 83.312 50.8))
  (stroke (width 0.2) (type solid)) (fill yes) (layer "F.Cu") (net 4))
 (gr_rect (start 78.546 33.447) (end 123.952 63.754) (stroke (width 0.05) (type default)) (fill no) (layer "Edge.Cuts"))
 (gr_circle (center 101.2444 40.132) (end 102.8446 40.1574) (stroke (width 0.05) (type default)) (fill no) (layer "Edge.Cuts"))
 (segment (start 115.634 37.683) (end 115.634 46.164) (width 0.635) (layer "F.Cu") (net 1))
 (segment (start 92.456 56.896) (end 92.456 49.53) (width 0.635) (layer "F.Cu") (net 1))
 (segment (start 105.427 36.085) (end 108.712 39.37) (width 0.635) (layer "F.Cu") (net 1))
 (segment (start 111.672 50.379) (end 111.165 50.379) (width 0.635) (layer "F.Cu") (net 1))
 (segment (start 111.672 50.126) (end 111.672 50.379) (width 0.508) (layer "F.Cu") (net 1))
 (segment (start 111.165 50.379) (end 101.6 59.944) (width 0.635) (layer "F.Cu") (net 1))
 (segment (start 101.6 59.944) (end 95.504 59.944) (width 0.635) (layer "F.Cu") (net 1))
 (segment (start 115.634 46.164) (end 111.672 50.126) (width 0.635) (layer "F.Cu") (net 1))
 (segment (start 110.323 50.379) (end 111.672 50.379) (width 0.635) (layer "F.Cu") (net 1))
 (segment (start 107.696 43.942) (end 107.696 47.752) (width 0.635) (layer "F.Cu") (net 1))
 (segment (start 108.712 42.926) (end 107.696 43.942) (width 0.635) (layer "F.Cu") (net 1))
 (segment (start 107.696 47.752) (end 110.323 50.379) (width 0.635) (layer "F.Cu") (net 1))
 (segment (start 108.712 39.37) (end 108.712 42.926) (width 0.635) (layer "F.Cu") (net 1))
 (segment (start 95.504 59.944) (end 92.456 56.896) (width 0.635) (layer "F.Cu") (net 1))
 (segment (start 104.951 36.085) (end 105.427 36.085) (width 0.635) (layer "F.Cu") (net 1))
 (segment (start 92.456 49.53) (end 89.916 46.99) (width 0.508) (layer "F.Cu") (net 1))
 (segment (start 117.217 56.519) (end 121.832 51.904) (width 0.635) (layer "F.Cu") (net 2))
 (segment (start 120.634 37.683) (end 120.634 44.688) (width 0.635) (layer "F.Cu") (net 2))
 (segment (start 121.92 50.291) (end 121.832 50.379) (width 0.508) (layer "F.Cu") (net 2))
 (segment (start 120.634 44.688) (end 121.92 45.974) (width 0.635) (layer "F.Cu") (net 2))
 (segment (start 121.832 51.904) (end 121.832 50.379) (width 0.635) (layer "F.Cu") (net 2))
 (segment (start 121.92 45.974) (end 121.92 50.291) (width 0.635) (layer "F.Cu") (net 2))
 (segment (start 117.217 59.445) (end 117.217 56.519) (width 0.635) (layer "F.Cu") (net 2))
 (segment (start 101.092 55.626) (end 98.933 57.785) (width 0.508) (layer "F.Cu") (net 8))
 (segment (start 100.484 47.291) (end 101.092 47.899) (width 0.508) (layer "F.Cu") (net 8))
 (segment (start 101.092 47.899) (end 101.092 55.626) (width 0.508) (layer "F.Cu") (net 8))
 (segment (start 99.722 47.291) (end 100.484 47.291) (width 0.508) (layer "F.Cu") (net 8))
 (segment (start 96.393 57.775) (end 94.887 56.269) (width 0.508) (layer "F.Cu") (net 9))
 (segment (start 94.887 56.269) (end 94.887 52.899) (width 0.508) (layer "F.Cu") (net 9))
 (segment (start 95.534 44.751) (end 94.535 44.751) (width 0.381) (layer "F.Cu") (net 4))
 (segment (start 93.472 43.688) (end 93.472 41.148) (width 0.381) (layer "F.Cu") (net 4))
 (segment (start 85.907 55.502) (end 84.207 55.502) (width 0.381) (layer "F.Cu") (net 4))
 (segment (start 110.549 45.759) (end 111.506 44.802) (width 0.508) (layer "F.Cu") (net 4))
 (segment (start 90.678 36.576) (end 92.964 36.576) (width 0.381) (layer "F.Cu") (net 4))
 (segment (start 110.401 59.347) (end 112.522 61.468) (width 0.381) (layer "F.Cu") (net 4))
 (segment (start 111.506 44.802) (end 111.485 44.781) (width 0.508) (layer "F.Cu") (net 4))
 (segment (start 102.411 35.609) (end 102.411 36.085) (width 0.381) (layer "F.Cu") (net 4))
 (segment (start 85.907 56.189) (end 90.678 60.96) (width 0.381) (layer "F.Cu") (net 4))
 (segment (start 102.411 36.085) (end 104.206 34.29) (width 0.381) (layer "F.Cu") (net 4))
 (segment (start 84.207 55.502) (end 81.207 52.502) (width 0.381) (layer "F.Cu") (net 4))
 (segment (start 92.964 36.576) (end 95.4015 34.1385) (width 0.381) (layer "F.Cu") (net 4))
 (segment (start 79.502 50.797) (end 79.502 41.656) (width 0.635) (layer "F.Cu") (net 4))
 (segment (start 100.9405 34.1385) (end 102.411 35.609) (width 0.381) (layer "F.Cu") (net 4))
 (segment (start 117.734 61.468) (end 119.757 59.445) (width 0.381) (layer "F.Cu") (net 4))
 (segment (start 95.4015 34.1385) (end 100.9405 34.1385) (width 0.381) (layer "F.Cu") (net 4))
 (segment (start 94.535 44.751) (end 93.472 43.688) (width 0.381) (layer "F.Cu") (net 4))
 (segment (start 111.485 44.781) (end 111.485 40.133) (width 0.508) (layer "F.Cu") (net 4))
 (segment (start 112.522 61.468) (end 117.734 61.468) (width 0.381) (layer "F.Cu") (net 4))
 (segment (start 93.472 41.148) (end 92.202 39.878) (width 0.381) (layer "F.Cu") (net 4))
 (segment (start 109.365 59.347) (end 110.401 59.347) (width 0.381) (layer "F.Cu") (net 4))
 (segment (start 104.206 34.29) (end 106.172 34.29) (width 0.381) (layer "F.Cu") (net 4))
 (segment (start 85.907 55.502) (end 85.907 56.189) (width 0.381) (layer "F.Cu") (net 4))
 (segment (start 100.484 43.481) (end 98.8568 41.8538) (width 0.381) (layer "F.Cu") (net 7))
 (segment (start 98.8568 41.8538) (end 98.8568 37.0992) (width 0.381) (layer "F.Cu") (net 7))
 (segment (start 98.8568 37.0992) (end 99.871 36.085) (width 0.381) (layer "F.Cu") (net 7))
 (segment (start 96.52 42.495) (end 96.52 36.896) (width 0.381) (layer "F.Cu") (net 6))
 (segment (start 96.52 36.896) (end 97.331 36.085) (width 0.381) (layer "F.Cu") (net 6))
 (segment (start 94.772 43.481) (end 95.534 43.481) (width 0.381) (layer "F.Cu") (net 6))
 (segment (start 95.534 43.481) (end 96.52 42.495) (width 0.381) (layer "F.Cu") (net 6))
 (segment (start 109.365 57.347) (end 108.068 57.347) (width 0.508) (layer "F.Cu") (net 3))
 (segment (start 114.677 59.445) (end 112.579 57.347) (width 0.508) (layer "F.Cu") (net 3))
 (segment (start 108.068 57.347) (end 104.938 60.477) (width 0.508) (layer "F.Cu") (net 3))
 (segment (start 112.579 57.347) (end 109.365 57.347) (width 0.508) (layer "F.Cu") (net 3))
 (segment (start 101.458999 46.021) (end 104.938 49.500001) (width 0.381) (layer "F.Cu") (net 11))
 (segment (start 100.484 46.021) (end 101.458999 46.021) (width 0.381) (layer "F.Cu") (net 11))
 (segment (start 104.938 49.500001) (end 104.938 50.317) (width 0.381) (layer "F.Cu") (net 11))
 (segment (start 102.155 44.751) (end 103.163 45.759) (width 0.381) (layer "F.Cu") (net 5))
 (segment (start 104.549 42.069) (end 106.485 40.133) (width 0.508) (layer "F.Cu") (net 5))
 (segment (start 103.163 45.759) (end 104.549 45.759) (width 0.381) (layer "F.Cu") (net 5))
 (segment (start 100.484 44.751) (end 102.155 44.751) (width 0.381) (layer "F.Cu") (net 5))
 (segment (start 104.549 45.759) (end 104.549 42.069) (width 0.508) (layer "F.Cu") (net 5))
 (segment (start 92.456 41.91) (end 91.44 40.894) (width 0.381) (layer "F.Cu") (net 10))
 (segment (start 91.44 40.894) (end 83.115 40.894) (width 0.381) (layer "F.Cu") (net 10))
 (segment (start 92.456 44.45) (end 92.456 41.91) (width 0.381) (layer "F.Cu") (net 10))
 (segment (start 94.027 46.021) (end 92.456 44.45) (width 0.381) (layer "F.Cu") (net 10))
 (segment (start 83.115 40.894) (end 81.062 42.947) (width 0.381) (layer "F.Cu") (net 10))
 (segment (start 95.534 46.021) (end 94.027 46.021) (width 0.381) (layer "F.Cu") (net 10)))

